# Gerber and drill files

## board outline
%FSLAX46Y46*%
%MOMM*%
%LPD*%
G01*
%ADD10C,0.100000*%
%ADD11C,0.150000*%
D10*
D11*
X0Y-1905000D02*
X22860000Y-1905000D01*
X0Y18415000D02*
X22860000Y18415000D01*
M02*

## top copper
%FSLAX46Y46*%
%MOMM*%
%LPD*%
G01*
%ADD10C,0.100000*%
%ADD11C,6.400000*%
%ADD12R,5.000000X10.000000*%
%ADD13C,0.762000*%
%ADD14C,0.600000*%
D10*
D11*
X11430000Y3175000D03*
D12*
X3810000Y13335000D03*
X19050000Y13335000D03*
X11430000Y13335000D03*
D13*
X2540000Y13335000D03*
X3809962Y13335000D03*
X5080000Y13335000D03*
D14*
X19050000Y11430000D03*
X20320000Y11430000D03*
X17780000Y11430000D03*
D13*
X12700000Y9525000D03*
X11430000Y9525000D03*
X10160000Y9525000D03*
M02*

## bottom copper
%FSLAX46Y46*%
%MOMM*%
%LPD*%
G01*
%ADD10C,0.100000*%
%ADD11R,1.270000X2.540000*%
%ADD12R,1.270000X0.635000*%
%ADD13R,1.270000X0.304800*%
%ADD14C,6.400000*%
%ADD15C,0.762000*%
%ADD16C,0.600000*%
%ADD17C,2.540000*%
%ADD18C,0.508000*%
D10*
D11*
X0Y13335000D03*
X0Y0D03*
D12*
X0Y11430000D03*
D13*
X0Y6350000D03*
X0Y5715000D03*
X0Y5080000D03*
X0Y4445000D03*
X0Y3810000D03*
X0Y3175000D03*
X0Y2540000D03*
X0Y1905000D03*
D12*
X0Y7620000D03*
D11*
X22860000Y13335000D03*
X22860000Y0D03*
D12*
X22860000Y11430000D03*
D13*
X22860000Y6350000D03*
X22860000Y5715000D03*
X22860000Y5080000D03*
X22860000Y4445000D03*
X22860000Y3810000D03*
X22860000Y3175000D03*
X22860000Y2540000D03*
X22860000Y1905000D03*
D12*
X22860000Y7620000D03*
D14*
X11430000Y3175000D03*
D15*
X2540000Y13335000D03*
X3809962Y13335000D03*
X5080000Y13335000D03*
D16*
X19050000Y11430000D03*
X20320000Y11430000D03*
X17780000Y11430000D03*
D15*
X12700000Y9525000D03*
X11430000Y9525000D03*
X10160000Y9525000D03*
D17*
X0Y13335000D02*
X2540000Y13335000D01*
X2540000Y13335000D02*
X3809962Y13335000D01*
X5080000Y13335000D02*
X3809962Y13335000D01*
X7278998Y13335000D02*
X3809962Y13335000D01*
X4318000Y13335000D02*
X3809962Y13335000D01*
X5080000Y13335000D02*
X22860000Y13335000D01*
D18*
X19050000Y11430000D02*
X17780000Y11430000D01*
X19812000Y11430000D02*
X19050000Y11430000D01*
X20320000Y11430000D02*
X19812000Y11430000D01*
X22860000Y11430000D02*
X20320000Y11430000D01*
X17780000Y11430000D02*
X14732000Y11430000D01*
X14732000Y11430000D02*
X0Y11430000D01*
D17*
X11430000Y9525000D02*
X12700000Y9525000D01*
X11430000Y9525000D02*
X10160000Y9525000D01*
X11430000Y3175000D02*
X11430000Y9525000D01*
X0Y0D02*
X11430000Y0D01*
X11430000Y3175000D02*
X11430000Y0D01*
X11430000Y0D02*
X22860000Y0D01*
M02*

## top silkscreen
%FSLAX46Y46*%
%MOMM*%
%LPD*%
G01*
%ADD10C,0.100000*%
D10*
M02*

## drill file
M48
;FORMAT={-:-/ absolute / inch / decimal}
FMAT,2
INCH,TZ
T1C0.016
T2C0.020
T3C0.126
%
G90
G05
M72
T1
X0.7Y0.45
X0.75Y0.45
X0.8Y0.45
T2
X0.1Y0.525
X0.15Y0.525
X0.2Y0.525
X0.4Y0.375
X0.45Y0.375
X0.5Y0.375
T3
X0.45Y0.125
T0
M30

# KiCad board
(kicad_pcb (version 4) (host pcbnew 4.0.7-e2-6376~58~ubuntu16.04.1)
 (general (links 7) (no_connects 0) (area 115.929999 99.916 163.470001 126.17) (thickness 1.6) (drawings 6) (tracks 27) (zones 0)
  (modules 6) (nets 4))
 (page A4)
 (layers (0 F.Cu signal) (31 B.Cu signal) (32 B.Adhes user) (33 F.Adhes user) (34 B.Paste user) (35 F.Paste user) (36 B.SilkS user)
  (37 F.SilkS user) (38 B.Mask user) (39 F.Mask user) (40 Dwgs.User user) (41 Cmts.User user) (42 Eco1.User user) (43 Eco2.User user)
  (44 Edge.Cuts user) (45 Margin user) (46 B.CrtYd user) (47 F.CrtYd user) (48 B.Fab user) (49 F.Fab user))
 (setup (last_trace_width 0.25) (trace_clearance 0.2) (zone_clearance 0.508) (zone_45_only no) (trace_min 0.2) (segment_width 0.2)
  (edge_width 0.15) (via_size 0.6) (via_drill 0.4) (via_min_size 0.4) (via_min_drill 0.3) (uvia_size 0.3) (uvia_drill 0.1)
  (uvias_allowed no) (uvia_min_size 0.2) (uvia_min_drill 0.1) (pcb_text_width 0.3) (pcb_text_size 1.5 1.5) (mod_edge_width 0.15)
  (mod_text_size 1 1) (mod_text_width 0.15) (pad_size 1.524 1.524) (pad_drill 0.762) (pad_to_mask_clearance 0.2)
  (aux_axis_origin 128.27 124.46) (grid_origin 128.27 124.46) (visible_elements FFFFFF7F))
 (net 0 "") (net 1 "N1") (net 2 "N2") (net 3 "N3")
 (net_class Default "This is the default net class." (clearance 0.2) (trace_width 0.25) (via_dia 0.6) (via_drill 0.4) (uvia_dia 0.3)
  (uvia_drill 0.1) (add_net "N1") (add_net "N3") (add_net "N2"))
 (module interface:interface (layer F.Cu) (at 128.27 104.775)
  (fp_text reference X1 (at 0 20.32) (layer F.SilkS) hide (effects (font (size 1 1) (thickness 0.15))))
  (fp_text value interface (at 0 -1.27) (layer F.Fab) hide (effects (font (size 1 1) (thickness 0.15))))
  (pad 1 smd rect (at 0 4.445) (size 1.27 2.54) (layers B.Cu) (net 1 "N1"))
  (pad 2 smd rect (at 0 17.78) (size 1.27 2.54) (layers B.Cu) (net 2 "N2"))
  (pad 3 smd rect (at 0 6.35) (size 1.27 0.635) (layers B.Cu) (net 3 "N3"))
  (pad 5 smd rect (at 0 11.43) (size 1.27 0.3048) (layers B.Cu))
  (pad 6 smd rect (at 0 12.065) (size 1.27 0.3048) (layers B.Cu))
  (pad 7 smd rect (at 0 12.7) (size 1.27 0.3048) (layers B.Cu))
  (pad 8 smd rect (at 0 13.335) (size 1.27 0.3048) (layers B.Cu))
  (pad 9 smd rect (at 0 13.97) (size 1.27 0.3048) (layers B.Cu))
  (pad 10 smd rect (at 0 14.605) (size 1.27 0.3048) (layers B.Cu))
  (pad 11 smd rect (at 0 15.24) (size 1.27 0.3048) (layers B.Cu))
  (pad 12 smd rect (at 0 15.875) (size 1.27 0.3048) (layers B.Cu))
  (pad 4 smd rect (at 0 10.16) (size 1.27 0.635) (layers B.Cu)))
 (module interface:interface (layer F.Cu) (at 151.13 104.775)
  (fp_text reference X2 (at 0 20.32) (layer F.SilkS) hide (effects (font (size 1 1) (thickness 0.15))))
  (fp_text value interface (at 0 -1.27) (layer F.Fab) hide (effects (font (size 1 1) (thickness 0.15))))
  (pad 1 smd rect (at 0 4.445) (size 1.27 2.54) (layers B.Cu) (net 1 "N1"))
  (pad 2 smd rect (at 0 17.78) (size 1.27 2.54) (layers B.Cu) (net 2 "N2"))
  (pad 3 smd rect (at 0 6.35) (size 1.27 0.635) (layers B.Cu) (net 3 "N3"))
  (pad 5 smd rect (at 0 11.43) (size 1.27 0.3048) (layers B.Cu))
  (pad 6 smd rect (at 0 12.065) (size 1.27 0.3048) (layers B.Cu))
  (pad 7 smd rect (at 0 12.7) (size 1.27 0.3048) (layers B.Cu))
  (pad 8 smd rect (at 0 13.335) (size 1.27 0.3048) (layers B.Cu))
  (pad 9 smd rect (at 0 13.97) (size 1.27 0.3048) (layers B.Cu))
  (pad 10 smd rect (at 0 14.605) (size 1.27 0.3048) (layers B.Cu))
  (pad 11 smd rect (at 0 15.24) (size 1.27 0.3048) (layers B.Cu))
  (pad 12 smd rect (at 0 15.875) (size 1.27 0.3048) (layers B.Cu))
  (pad 4 smd rect (at 0 10.16) (size 1.27 0.635) (layers B.Cu)))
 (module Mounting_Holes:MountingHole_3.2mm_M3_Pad (layer F.Cu) (at 139.7 119.38)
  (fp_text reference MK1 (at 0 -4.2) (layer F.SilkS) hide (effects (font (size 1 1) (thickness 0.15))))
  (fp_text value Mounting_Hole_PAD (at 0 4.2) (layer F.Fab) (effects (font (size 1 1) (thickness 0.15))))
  (pad 1 thru_hole circle (at 0 0) (size 6.4 6.4) (drill 3.2) (layers *.Cu *.Mask) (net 2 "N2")))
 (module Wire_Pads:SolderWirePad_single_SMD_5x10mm (layer F.Cu) (at 132.08 109.22 180)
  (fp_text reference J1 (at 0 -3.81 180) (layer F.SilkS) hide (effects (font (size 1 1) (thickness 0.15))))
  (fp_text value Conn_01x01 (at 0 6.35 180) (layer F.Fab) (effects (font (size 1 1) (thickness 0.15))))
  (pad 1 smd rect (at 0 0 180) (size 5 10) (layers F.Cu F.Paste F.Mask) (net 1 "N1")))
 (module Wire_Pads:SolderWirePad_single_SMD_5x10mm (layer F.Cu) (at 147.32 109.22 180)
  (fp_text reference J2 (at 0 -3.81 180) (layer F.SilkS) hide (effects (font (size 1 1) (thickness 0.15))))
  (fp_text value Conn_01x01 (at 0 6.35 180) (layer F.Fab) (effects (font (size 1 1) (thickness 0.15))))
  (pad 1 smd rect (at 0 0 180) (size 5 10) (layers F.Cu F.Paste F.Mask) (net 3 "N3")))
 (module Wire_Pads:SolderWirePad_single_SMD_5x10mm (layer F.Cu) (at 139.7 109.22)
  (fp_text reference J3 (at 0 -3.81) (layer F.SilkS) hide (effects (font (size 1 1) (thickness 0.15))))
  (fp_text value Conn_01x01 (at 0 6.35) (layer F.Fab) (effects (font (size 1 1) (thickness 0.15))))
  (pad 1 smd rect (at 0 0) (size 5 10) (layers F.Cu F.Paste F.Mask) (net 2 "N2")))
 (gr_line (start 128.27 124.46) (end 151.13 124.46) (layer Edge.Cuts) (width 0.15))
 (gr_line (start 128.27 104.14) (end 151.13 104.14) (layer Edge.Cuts) (width 0.15))
 (segment (start 128.27 109.22) (end 130.81 109.22) (width 2.54) (layer B.Cu) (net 1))
 (segment (start 130.81 109.22) (end 132.079962 109.22) (width 2.54) (layer B.Cu) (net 1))
 (via (at 130.81 109.22) (size 0.762) (drill 0.508) (layers F.Cu B.Cu) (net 1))
 (segment (start 133.35 109.22) (end 132.079962 109.22) (width 2.54) (layer B.Cu) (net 1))
 (segment (start 135.548998 109.22) (end 132.079962 109.22) (width 2.54) (layer B.Cu) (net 1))
 (segment (start 132.588 109.22) (end 132.079962 109.22) (width 2.54) (layer B.Cu) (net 1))
 (via (at 132.079962 109.22) (size 0.762) (drill 0.508) (layers F.Cu B.Cu) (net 1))
 (segment (start 133.35 109.22) (end 151.13 109.22) (width 2.54) (layer B.Cu) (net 1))
 (via (at 133.35 109.22) (size 0.762) (drill 0.508) (layers F.Cu B.Cu) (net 1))
 (segment (start 147.32 111.125) (end 146.05 111.125) (width 0.508) (layer B.Cu) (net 3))
 (segment (start 148.082 111.125) (end 147.32 111.125) (width 0.508) (layer B.Cu) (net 3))
 (via (at 147.32 111.125) (size 0.6) (drill 0.4) (layers F.Cu B.Cu) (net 3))
 (segment (start 148.59 111.125) (end 148.082 111.125) (width 0.508) (layer B.Cu) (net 3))
 (via (at 148.59 111.125) (size 0.6) (drill 0.4) (layers F.Cu B.Cu) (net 3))
 (segment (start 151.13 111.125) (end 148.59 111.125) (width 0.508) (layer B.Cu) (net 3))
 (segment (start 146.05 111.125) (end 143.002 111.125) (width 0.508) (layer B.Cu) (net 3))
 (via (at 146.05 111.125) (size 0.6) (drill 0.4) (layers F.Cu B.Cu) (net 3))
 (segment (start 143.002 111.125) (end 128.27 111.125) (width 0.508) (layer B.Cu) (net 3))
 (via (at 140.97 113.03) (size 0.762) (drill 0.508) (layers F.Cu B.Cu) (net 2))
 (via (at 139.7 113.03) (size 0.762) (drill 0.508) (layers F.Cu B.Cu) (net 2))
 (via (at 138.43 113.03) (size 0.762) (drill 0.508) (layers F.Cu B.Cu) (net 2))
 (segment (start 139.7 113.03) (end 140.97 113.03) (width 2.54) (layer B.Cu) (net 2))
 (segment (start 139.7 113.03) (end 138.43 113.03) (width 2.54) (layer B.Cu) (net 2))
 (segment (start 139.7 119.38) (end 139.7 113.03) (width 2.54) (layer B.Cu) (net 2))
 (segment (start 128.27 122.555) (end 139.7 122.555) (width 2.54) (layer B.Cu) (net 2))
 (segment (start 139.7 119.38) (end 139.7 122.555) (width 2.54) (layer B.Cu) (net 2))
 (segment (start 139.7 122.555) (end 151.13 122.555) (width 2.54) (layer B.Cu) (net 2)))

